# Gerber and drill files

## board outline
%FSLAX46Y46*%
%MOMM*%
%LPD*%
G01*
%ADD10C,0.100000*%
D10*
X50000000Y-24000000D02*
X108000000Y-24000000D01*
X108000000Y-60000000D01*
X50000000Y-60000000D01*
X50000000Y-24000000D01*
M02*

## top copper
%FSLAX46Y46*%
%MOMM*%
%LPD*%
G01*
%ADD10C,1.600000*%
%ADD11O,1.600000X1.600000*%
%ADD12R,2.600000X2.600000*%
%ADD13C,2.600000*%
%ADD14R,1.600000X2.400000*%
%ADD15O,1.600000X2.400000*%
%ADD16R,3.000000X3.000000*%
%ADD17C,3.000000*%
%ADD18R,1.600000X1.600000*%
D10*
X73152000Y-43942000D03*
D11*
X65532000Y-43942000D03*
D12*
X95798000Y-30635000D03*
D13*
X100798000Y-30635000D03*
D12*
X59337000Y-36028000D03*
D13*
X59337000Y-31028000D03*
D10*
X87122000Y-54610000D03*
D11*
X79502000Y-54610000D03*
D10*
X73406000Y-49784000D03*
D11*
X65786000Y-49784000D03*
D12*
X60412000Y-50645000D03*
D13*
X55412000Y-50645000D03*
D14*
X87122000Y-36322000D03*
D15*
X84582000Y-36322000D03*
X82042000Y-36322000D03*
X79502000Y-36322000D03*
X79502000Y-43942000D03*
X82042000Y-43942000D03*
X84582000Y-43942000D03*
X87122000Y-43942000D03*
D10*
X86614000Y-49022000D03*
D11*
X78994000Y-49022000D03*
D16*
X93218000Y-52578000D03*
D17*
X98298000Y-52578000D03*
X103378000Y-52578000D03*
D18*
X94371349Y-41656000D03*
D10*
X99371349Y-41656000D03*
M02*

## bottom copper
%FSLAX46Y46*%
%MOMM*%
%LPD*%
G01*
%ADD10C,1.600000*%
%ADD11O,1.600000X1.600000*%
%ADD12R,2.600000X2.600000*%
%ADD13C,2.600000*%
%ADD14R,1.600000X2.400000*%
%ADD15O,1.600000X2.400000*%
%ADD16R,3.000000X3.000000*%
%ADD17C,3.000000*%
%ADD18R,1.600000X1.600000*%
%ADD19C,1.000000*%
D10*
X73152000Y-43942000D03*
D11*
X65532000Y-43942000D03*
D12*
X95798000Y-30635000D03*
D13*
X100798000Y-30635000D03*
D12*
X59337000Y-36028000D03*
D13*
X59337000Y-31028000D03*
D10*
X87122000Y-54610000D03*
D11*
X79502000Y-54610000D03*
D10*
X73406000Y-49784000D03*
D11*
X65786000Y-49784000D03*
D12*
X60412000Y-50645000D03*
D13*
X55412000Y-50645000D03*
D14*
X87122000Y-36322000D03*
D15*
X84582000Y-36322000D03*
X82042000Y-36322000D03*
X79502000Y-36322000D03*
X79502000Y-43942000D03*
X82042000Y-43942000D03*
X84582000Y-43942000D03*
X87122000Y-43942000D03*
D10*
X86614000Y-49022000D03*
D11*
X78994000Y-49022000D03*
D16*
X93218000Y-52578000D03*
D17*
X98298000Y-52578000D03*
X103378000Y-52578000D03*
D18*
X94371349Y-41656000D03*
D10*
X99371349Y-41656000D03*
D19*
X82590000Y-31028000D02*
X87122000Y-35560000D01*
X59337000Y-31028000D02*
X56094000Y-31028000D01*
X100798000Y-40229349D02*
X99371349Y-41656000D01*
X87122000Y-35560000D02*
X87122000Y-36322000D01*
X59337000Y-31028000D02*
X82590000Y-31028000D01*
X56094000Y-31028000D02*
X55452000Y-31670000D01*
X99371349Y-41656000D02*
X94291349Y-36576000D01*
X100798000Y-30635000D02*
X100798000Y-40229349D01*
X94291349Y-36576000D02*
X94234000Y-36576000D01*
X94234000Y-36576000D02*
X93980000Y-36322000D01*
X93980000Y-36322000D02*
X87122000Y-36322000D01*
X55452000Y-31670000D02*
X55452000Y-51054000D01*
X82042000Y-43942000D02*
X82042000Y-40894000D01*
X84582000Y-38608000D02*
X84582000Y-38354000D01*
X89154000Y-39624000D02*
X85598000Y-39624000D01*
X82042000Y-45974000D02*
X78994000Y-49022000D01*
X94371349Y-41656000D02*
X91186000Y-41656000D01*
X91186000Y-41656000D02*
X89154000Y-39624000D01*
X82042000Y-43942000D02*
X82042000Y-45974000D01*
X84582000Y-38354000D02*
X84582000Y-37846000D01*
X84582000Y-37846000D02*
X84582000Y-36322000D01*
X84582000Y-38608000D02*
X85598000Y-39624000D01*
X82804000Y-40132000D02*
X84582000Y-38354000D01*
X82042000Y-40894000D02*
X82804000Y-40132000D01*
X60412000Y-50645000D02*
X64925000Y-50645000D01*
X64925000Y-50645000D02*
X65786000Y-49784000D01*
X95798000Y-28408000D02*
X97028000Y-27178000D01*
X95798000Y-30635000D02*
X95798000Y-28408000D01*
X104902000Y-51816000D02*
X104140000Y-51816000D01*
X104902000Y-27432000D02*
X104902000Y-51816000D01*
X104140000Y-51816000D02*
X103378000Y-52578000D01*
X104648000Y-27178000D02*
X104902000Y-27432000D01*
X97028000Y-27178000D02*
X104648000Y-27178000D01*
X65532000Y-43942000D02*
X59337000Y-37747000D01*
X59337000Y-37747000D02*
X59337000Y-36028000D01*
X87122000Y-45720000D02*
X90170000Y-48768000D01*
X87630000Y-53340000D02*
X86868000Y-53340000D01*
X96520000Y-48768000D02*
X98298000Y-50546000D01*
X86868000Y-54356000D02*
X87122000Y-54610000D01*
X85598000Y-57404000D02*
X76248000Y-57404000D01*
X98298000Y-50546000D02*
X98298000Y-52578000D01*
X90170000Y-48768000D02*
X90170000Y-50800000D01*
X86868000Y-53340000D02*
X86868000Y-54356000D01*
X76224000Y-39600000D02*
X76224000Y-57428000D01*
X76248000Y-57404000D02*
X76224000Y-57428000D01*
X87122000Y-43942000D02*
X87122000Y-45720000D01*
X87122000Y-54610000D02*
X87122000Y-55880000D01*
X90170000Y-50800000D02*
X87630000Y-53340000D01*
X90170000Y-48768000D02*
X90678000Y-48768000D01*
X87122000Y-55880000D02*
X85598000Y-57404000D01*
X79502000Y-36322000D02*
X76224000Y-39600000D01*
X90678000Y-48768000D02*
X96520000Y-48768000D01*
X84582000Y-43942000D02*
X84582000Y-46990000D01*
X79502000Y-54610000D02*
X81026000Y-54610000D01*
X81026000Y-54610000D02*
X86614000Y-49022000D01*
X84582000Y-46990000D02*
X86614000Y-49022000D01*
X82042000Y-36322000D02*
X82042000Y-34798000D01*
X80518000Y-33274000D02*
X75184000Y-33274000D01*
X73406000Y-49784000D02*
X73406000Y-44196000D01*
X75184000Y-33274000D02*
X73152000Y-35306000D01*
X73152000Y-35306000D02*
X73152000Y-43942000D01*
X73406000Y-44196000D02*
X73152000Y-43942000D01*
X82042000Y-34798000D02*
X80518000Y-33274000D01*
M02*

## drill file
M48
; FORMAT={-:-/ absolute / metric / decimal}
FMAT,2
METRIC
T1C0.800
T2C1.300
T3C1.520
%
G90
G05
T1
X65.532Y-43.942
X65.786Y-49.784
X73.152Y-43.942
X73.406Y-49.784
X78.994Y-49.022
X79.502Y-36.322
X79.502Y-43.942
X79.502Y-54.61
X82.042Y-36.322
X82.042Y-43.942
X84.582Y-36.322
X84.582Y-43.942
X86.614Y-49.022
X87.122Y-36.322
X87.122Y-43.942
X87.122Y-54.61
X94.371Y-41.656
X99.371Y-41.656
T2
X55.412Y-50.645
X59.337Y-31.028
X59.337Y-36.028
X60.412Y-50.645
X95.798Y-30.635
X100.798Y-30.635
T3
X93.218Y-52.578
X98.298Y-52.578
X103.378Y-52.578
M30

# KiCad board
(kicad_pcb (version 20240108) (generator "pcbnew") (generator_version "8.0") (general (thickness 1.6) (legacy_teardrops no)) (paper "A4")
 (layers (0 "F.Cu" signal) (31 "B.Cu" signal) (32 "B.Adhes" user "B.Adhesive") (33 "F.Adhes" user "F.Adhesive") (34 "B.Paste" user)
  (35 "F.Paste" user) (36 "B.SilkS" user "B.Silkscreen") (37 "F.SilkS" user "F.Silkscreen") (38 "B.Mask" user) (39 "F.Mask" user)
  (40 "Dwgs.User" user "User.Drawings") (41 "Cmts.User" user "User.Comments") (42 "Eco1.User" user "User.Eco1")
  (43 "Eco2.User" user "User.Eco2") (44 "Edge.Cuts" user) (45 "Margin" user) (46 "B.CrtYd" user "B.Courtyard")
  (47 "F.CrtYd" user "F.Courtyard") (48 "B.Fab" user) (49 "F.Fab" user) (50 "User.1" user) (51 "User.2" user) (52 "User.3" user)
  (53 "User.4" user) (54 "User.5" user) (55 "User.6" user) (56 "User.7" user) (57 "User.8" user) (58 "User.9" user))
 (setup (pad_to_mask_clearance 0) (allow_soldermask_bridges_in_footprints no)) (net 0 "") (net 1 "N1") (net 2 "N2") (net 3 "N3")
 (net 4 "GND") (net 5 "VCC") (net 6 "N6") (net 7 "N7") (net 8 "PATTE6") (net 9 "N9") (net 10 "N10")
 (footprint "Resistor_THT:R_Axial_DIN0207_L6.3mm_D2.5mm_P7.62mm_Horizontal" (layer "F.Cu") (at 73.152 43.942 180)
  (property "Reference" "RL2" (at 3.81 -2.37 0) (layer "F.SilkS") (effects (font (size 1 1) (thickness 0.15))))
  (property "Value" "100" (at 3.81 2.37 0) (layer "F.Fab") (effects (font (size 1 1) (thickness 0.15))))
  (pad "1" thru_hole circle (at 0 0 180) (size 1.6 1.6) (drill 0.8) (layers "*.Cu" "*.Mask") (remove_unused_layers no) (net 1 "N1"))
  (pad "2" thru_hole oval (at 7.62 0 180) (size 1.6 1.6) (drill 0.8) (layers "*.Cu" "*.Mask") (remove_unused_layers no) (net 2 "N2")))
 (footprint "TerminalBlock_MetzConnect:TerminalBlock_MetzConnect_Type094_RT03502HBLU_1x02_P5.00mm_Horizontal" (layer "F.Cu")
  (at 95.798 30.635)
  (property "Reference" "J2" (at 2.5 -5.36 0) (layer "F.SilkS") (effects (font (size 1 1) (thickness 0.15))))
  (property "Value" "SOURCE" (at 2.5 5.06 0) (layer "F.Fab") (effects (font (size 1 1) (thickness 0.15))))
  (pad "1" thru_hole rect (at 0 0) (size 2.6 2.6) (drill 1.3) (layers "*.Cu" "*.Mask") (remove_unused_layers no) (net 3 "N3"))
  (pad "2" thru_hole circle (at 5 0) (size 2.6 2.6) (drill 1.3) (layers "*.Cu" "*.Mask") (remove_unused_layers no) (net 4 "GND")))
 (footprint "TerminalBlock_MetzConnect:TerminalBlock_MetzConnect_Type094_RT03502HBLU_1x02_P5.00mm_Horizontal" (layer "F.Cu")
  (at 59.337 36.028 90)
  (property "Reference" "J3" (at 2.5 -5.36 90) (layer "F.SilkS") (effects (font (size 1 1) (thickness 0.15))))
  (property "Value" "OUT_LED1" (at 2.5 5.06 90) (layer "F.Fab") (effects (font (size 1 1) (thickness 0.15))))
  (pad "1" thru_hole rect (at 0 0 90) (size 2.6 2.6) (drill 1.3) (layers "*.Cu" "*.Mask") (remove_unused_layers no) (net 2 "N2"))
  (pad "2" thru_hole circle (at 5 0 90) (size 2.6 2.6) (drill 1.3) (layers "*.Cu" "*.Mask") (remove_unused_layers no) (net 4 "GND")))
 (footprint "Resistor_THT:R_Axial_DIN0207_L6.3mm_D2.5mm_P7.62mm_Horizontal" (layer "F.Cu") (at 87.122 54.61 180)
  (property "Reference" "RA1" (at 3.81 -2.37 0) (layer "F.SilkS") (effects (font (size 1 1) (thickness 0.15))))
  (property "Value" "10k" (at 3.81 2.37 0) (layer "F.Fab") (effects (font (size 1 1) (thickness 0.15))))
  (pad "1" thru_hole circle (at 0 0 180) (size 1.6 1.6) (drill 0.8) (layers "*.Cu" "*.Mask") (remove_unused_layers no) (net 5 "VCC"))
  (pad "2" thru_hole oval (at 7.62 0 180) (size 1.6 1.6) (drill 0.8) (layers "*.Cu" "*.Mask") (remove_unused_layers no) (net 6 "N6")))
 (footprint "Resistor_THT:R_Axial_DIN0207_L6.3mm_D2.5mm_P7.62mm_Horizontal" (layer "F.Cu") (at 73.406 49.784 180)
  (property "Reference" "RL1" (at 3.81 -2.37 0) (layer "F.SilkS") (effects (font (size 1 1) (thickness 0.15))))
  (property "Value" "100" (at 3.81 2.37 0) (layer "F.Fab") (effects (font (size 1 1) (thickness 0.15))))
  (pad "1" thru_hole circle (at 0 0 180) (size 1.6 1.6) (drill 0.8) (layers "*.Cu" "*.Mask") (remove_unused_layers no) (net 1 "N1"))
  (pad "2" thru_hole oval (at 7.62 0 180) (size 1.6 1.6) (drill 0.8) (layers "*.Cu" "*.Mask") (remove_unused_layers no) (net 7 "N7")))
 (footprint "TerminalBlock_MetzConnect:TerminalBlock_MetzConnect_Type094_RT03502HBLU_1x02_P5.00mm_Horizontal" (layer "F.Cu")
  (at 60.412 50.645 180)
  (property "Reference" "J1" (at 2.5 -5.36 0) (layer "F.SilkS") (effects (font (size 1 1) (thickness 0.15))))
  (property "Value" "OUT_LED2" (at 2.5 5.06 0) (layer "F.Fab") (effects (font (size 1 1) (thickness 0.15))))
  (pad "1" thru_hole rect (at 0 0 180) (size 2.6 2.6) (drill 1.3) (layers "*.Cu" "*.Mask") (remove_unused_layers no) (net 7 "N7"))
  (pad "2" thru_hole circle (at 5 0 180) (size 2.6 2.6) (drill 1.3) (layers "*.Cu" "*.Mask") (remove_unused_layers no) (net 4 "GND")))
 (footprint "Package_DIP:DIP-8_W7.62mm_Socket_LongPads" (layer "F.Cu") (at 87.122 36.322 -90)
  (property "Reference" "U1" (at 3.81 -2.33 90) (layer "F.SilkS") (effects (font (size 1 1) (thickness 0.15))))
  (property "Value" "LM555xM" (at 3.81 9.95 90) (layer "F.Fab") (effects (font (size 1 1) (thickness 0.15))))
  (pad "1" thru_hole rect (at 0 0 270) (size 2.4 1.6) (drill 0.8) (layers "*.Cu" "*.Mask") (remove_unused_layers no) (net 4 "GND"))
  (pad "2" thru_hole oval (at 0 2.54 270) (size 2.4 1.6) (drill 0.8) (layers "*.Cu" "*.Mask") (remove_unused_layers no) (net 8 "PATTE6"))
  (pad "3" thru_hole oval (at 0 5.08 270) (size 2.4 1.6) (drill 0.8) (layers "*.Cu" "*.Mask") (remove_unused_layers no) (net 1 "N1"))
  (pad "4" thru_hole oval (at 0 7.62 270) (size 2.4 1.6) (drill 0.8) (layers "*.Cu" "*.Mask") (remove_unused_layers no) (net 5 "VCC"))
  (pad "5" thru_hole oval (at 7.62 7.62 270) (size 2.4 1.6) (drill 0.8) (layers "*.Cu" "*.Mask") (remove_unused_layers no) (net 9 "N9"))
  (pad "6" thru_hole oval (at 7.62 5.08 270) (size 2.4 1.6) (drill 0.8) (layers "*.Cu" "*.Mask") (remove_unused_layers no) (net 8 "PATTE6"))
  (pad "7" thru_hole oval (at 7.62 2.54 270) (size 2.4 1.6) (drill 0.8) (layers "*.Cu" "*.Mask") (remove_unused_layers no) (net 6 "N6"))
  (pad "8" thru_hole oval (at 7.62 0 270) (size 2.4 1.6) (drill 0.8) (layers "*.Cu" "*.Mask") (remove_unused_layers no) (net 5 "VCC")))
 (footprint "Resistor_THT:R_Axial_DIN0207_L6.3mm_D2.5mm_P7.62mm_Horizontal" (layer "F.Cu") (at 86.614 49.022 180)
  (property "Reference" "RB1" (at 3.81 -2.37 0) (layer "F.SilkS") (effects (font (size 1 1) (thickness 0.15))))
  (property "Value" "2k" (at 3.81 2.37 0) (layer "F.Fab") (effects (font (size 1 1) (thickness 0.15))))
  (pad "1" thru_hole circle (at 0 0 180) (size 1.6 1.6) (drill 0.8) (layers "*.Cu" "*.Mask") (remove_unused_layers no) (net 6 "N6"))
  (pad "2" thru_hole oval (at 7.62 0 180) (size 1.6 1.6) (drill 0.8) (layers "*.Cu" "*.Mask") (remove_unused_layers no) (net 8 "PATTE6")))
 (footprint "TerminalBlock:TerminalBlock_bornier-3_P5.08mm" (layer "F.Cu") (at 93.218 52.578)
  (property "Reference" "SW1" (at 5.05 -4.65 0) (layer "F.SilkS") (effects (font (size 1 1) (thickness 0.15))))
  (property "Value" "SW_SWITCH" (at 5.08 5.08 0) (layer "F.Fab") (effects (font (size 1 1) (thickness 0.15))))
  (pad "1" thru_hole rect (at 0 0) (size 3 3) (drill 1.52) (layers "*.Cu" "*.Mask") (remove_unused_layers no) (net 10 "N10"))
  (pad "2" thru_hole circle (at 5.08 0) (size 3 3) (drill 1.52) (layers "*.Cu" "*.Mask") (remove_unused_layers no) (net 5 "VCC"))
  (pad "3" thru_hole circle (at 10.16 0) (size 3 3) (drill 1.52) (layers "*.Cu" "*.Mask") (remove_unused_layers no) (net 3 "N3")))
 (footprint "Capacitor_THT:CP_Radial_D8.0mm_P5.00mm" (layer "F.Cu") (at 94.371349 41.656)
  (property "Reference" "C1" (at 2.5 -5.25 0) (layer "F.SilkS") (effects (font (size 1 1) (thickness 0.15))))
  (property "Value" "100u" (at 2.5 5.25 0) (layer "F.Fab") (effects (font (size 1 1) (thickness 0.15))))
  (pad "1" thru_hole rect (at 0 0) (size 1.6 1.6) (drill 0.8) (layers "*.Cu" "*.Mask") (remove_unused_layers no) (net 8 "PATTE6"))
  (pad "2" thru_hole circle (at 5 0) (size 1.6 1.6) (drill 0.8) (layers "*.Cu" "*.Mask") (remove_unused_layers no) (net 4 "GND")))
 (gr_rect (start 50 24) (end 108 60) (stroke (width 0.1) (type default)) (fill none) (layer "Edge.Cuts"))
 (segment (start 82.59 31.028) (end 87.122 35.56) (width 1) (layer "B.Cu") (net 4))
 (segment (start 59.337 31.028) (end 56.094 31.028) (width 1) (layer "B.Cu") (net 4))
 (segment (start 100.798 40.229349) (end 99.371349 41.656) (width 1) (layer "B.Cu") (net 4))
 (segment (start 87.122 35.56) (end 87.122 36.322) (width 1) (layer "B.Cu") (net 4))
 (segment (start 59.337 31.028) (end 82.59 31.028) (width 1) (layer "B.Cu") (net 4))
 (segment (start 56.094 31.028) (end 55.452 31.67) (width 1) (layer "B.Cu") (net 4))
 (segment (start 99.371349 41.656) (end 94.291349 36.576) (width 1) (layer "B.Cu") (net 4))
 (segment (start 100.798 30.635) (end 100.798 40.229349) (width 1) (layer "B.Cu") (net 4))
 (segment (start 94.291349 36.576) (end 94.234 36.576) (width 1) (layer "B.Cu") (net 4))
 (segment (start 94.234 36.576) (end 93.98 36.322) (width 1) (layer "B.Cu") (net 4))
 (segment (start 93.98 36.322) (end 87.122 36.322) (width 1) (layer "B.Cu") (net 4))
 (segment (start 55.452 31.67) (end 55.452 51.054) (width 1) (layer "B.Cu") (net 4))
 (segment (start 82.042 43.942) (end 82.042 40.894) (width 1) (layer "B.Cu") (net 8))
 (segment (start 84.582 38.608) (end 84.582 38.354) (width 1) (layer "B.Cu") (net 8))
 (segment (start 89.154 39.624) (end 85.598 39.624) (width 1) (layer "B.Cu") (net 8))
 (segment (start 82.042 45.974) (end 78.994 49.022) (width 1) (layer "B.Cu") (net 8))
 (segment (start 94.371349 41.656) (end 91.186 41.656) (width 1) (layer "B.Cu") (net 8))
 (segment (start 91.186 41.656) (end 89.154 39.624) (width 1) (layer "B.Cu") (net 8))
 (segment (start 82.042 43.942) (end 82.042 45.974) (width 1) (layer "B.Cu") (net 8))
 (segment (start 84.582 38.354) (end 84.582 37.846) (width 1) (layer "B.Cu") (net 8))
 (segment (start 84.582 37.846) (end 84.582 36.322) (width 1) (layer "B.Cu") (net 8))
 (segment (start 84.582 38.608) (end 85.598 39.624) (width 1) (layer "B.Cu") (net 8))
 (segment (start 82.804 40.132) (end 84.582 38.354) (width 1) (layer "B.Cu") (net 8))
 (segment (start 82.042 40.894) (end 82.804 40.132) (width 1) (layer "B.Cu") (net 8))
 (segment (start 60.412 50.645) (end 64.925 50.645) (width 1) (layer "B.Cu") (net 7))
 (segment (start 64.925 50.645) (end 65.786 49.784) (width 1) (layer "B.Cu") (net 7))
 (segment (start 95.798 28.408) (end 97.028 27.178) (width 1) (layer "B.Cu") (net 3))
 (segment (start 95.798 30.635) (end 95.798 28.408) (width 1) (layer "B.Cu") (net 3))
 (segment (start 104.902 51.816) (end 104.14 51.816) (width 1) (layer "B.Cu") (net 3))
 (segment (start 104.902 27.432) (end 104.902 51.816) (width 1) (layer "B.Cu") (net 3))
 (segment (start 104.14 51.816) (end 103.378 52.578) (width 1) (layer "B.Cu") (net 3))
 (segment (start 104.648 27.178) (end 104.902 27.432) (width 1) (layer "B.Cu") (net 3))
 (segment (start 97.028 27.178) (end 104.648 27.178) (width 1) (layer "B.Cu") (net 3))
 (segment (start 65.532 43.942) (end 59.337 37.747) (width 1) (layer "B.Cu") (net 2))
 (segment (start 59.337 37.747) (end 59.337 36.028) (width 1) (layer "B.Cu") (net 2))
 (segment (start 87.122 45.72) (end 90.17 48.768) (width 1) (layer "B.Cu") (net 5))
 (segment (start 87.63 53.34) (end 86.868 53.34) (width 1) (layer "B.Cu") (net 5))
 (segment (start 96.52 48.768) (end 98.298 50.546) (width 1) (layer "B.Cu") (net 5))
 (segment (start 86.868 54.356) (end 87.122 54.61) (width 1) (layer "B.Cu") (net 5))
 (segment (start 85.598 57.404) (end 76.248 57.404) (width 1) (layer "B.Cu") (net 5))
 (segment (start 98.298 50.546) (end 98.298 52.578) (width 1) (layer "B.Cu") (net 5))
 (segment (start 90.17 48.768) (end 90.17 50.8) (width 1) (layer "B.Cu") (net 5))
 (segment (start 86.868 53.34) (end 86.868 54.356) (width 1) (layer "B.Cu") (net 5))
 (segment (start 76.224 39.6) (end 76.224 57.428) (width 1) (layer "B.Cu") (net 5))
 (segment (start 76.248 57.404) (end 76.224 57.428) (width 1) (layer "B.Cu") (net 5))
 (segment (start 87.122 43.942) (end 87.122 45.72) (width 1) (layer "B.Cu") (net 5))
 (segment (start 87.122 54.61) (end 87.122 55.88) (width 1) (layer "B.Cu") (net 5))
 (segment (start 90.17 50.8) (end 87.63 53.34) (width 1) (layer "B.Cu") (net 5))
 (segment (start 90.17 48.768) (end 90.678 48.768) (width 1) (layer "B.Cu") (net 5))
 (segment (start 87.122 55.88) (end 85.598 57.404) (width 1) (layer "B.Cu") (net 5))
 (segment (start 79.502 36.322) (end 76.224 39.6) (width 1) (layer "B.Cu") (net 5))
 (segment (start 90.678 48.768) (end 96.52 48.768) (width 1) (layer "B.Cu") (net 5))
 (segment (start 84.582 43.942) (end 84.582 46.99) (width 1) (layer "B.Cu") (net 6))
 (segment (start 79.502 54.61) (end 81.026 54.61) (width 1) (layer "B.Cu") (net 6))
 (segment (start 81.026 54.61) (end 86.614 49.022) (width 1) (layer "B.Cu") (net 6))
 (segment (start 84.582 46.99) (end 86.614 49.022) (width 1) (layer "B.Cu") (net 6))
 (segment (start 82.042 36.322) (end 82.042 34.798) (width 1) (layer "B.Cu") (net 1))
 (segment (start 80.518 33.274) (end 75.184 33.274) (width 1) (layer "B.Cu") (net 1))
 (segment (start 73.406 49.784) (end 73.406 44.196) (width 1) (layer "B.Cu") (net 1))
 (segment (start 75.184 33.274) (end 73.152 35.306) (width 1) (layer "B.Cu") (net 1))
 (segment (start 73.152 35.306) (end 73.152 43.942) (width 1) (layer "B.Cu") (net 1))
 (segment (start 73.406 44.196) (end 73.152 43.942) (width 1) (layer "B.Cu") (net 1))
 (segment (start 82.042 34.798) (end 80.518 33.274) (width 1) (layer "B.Cu") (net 1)))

